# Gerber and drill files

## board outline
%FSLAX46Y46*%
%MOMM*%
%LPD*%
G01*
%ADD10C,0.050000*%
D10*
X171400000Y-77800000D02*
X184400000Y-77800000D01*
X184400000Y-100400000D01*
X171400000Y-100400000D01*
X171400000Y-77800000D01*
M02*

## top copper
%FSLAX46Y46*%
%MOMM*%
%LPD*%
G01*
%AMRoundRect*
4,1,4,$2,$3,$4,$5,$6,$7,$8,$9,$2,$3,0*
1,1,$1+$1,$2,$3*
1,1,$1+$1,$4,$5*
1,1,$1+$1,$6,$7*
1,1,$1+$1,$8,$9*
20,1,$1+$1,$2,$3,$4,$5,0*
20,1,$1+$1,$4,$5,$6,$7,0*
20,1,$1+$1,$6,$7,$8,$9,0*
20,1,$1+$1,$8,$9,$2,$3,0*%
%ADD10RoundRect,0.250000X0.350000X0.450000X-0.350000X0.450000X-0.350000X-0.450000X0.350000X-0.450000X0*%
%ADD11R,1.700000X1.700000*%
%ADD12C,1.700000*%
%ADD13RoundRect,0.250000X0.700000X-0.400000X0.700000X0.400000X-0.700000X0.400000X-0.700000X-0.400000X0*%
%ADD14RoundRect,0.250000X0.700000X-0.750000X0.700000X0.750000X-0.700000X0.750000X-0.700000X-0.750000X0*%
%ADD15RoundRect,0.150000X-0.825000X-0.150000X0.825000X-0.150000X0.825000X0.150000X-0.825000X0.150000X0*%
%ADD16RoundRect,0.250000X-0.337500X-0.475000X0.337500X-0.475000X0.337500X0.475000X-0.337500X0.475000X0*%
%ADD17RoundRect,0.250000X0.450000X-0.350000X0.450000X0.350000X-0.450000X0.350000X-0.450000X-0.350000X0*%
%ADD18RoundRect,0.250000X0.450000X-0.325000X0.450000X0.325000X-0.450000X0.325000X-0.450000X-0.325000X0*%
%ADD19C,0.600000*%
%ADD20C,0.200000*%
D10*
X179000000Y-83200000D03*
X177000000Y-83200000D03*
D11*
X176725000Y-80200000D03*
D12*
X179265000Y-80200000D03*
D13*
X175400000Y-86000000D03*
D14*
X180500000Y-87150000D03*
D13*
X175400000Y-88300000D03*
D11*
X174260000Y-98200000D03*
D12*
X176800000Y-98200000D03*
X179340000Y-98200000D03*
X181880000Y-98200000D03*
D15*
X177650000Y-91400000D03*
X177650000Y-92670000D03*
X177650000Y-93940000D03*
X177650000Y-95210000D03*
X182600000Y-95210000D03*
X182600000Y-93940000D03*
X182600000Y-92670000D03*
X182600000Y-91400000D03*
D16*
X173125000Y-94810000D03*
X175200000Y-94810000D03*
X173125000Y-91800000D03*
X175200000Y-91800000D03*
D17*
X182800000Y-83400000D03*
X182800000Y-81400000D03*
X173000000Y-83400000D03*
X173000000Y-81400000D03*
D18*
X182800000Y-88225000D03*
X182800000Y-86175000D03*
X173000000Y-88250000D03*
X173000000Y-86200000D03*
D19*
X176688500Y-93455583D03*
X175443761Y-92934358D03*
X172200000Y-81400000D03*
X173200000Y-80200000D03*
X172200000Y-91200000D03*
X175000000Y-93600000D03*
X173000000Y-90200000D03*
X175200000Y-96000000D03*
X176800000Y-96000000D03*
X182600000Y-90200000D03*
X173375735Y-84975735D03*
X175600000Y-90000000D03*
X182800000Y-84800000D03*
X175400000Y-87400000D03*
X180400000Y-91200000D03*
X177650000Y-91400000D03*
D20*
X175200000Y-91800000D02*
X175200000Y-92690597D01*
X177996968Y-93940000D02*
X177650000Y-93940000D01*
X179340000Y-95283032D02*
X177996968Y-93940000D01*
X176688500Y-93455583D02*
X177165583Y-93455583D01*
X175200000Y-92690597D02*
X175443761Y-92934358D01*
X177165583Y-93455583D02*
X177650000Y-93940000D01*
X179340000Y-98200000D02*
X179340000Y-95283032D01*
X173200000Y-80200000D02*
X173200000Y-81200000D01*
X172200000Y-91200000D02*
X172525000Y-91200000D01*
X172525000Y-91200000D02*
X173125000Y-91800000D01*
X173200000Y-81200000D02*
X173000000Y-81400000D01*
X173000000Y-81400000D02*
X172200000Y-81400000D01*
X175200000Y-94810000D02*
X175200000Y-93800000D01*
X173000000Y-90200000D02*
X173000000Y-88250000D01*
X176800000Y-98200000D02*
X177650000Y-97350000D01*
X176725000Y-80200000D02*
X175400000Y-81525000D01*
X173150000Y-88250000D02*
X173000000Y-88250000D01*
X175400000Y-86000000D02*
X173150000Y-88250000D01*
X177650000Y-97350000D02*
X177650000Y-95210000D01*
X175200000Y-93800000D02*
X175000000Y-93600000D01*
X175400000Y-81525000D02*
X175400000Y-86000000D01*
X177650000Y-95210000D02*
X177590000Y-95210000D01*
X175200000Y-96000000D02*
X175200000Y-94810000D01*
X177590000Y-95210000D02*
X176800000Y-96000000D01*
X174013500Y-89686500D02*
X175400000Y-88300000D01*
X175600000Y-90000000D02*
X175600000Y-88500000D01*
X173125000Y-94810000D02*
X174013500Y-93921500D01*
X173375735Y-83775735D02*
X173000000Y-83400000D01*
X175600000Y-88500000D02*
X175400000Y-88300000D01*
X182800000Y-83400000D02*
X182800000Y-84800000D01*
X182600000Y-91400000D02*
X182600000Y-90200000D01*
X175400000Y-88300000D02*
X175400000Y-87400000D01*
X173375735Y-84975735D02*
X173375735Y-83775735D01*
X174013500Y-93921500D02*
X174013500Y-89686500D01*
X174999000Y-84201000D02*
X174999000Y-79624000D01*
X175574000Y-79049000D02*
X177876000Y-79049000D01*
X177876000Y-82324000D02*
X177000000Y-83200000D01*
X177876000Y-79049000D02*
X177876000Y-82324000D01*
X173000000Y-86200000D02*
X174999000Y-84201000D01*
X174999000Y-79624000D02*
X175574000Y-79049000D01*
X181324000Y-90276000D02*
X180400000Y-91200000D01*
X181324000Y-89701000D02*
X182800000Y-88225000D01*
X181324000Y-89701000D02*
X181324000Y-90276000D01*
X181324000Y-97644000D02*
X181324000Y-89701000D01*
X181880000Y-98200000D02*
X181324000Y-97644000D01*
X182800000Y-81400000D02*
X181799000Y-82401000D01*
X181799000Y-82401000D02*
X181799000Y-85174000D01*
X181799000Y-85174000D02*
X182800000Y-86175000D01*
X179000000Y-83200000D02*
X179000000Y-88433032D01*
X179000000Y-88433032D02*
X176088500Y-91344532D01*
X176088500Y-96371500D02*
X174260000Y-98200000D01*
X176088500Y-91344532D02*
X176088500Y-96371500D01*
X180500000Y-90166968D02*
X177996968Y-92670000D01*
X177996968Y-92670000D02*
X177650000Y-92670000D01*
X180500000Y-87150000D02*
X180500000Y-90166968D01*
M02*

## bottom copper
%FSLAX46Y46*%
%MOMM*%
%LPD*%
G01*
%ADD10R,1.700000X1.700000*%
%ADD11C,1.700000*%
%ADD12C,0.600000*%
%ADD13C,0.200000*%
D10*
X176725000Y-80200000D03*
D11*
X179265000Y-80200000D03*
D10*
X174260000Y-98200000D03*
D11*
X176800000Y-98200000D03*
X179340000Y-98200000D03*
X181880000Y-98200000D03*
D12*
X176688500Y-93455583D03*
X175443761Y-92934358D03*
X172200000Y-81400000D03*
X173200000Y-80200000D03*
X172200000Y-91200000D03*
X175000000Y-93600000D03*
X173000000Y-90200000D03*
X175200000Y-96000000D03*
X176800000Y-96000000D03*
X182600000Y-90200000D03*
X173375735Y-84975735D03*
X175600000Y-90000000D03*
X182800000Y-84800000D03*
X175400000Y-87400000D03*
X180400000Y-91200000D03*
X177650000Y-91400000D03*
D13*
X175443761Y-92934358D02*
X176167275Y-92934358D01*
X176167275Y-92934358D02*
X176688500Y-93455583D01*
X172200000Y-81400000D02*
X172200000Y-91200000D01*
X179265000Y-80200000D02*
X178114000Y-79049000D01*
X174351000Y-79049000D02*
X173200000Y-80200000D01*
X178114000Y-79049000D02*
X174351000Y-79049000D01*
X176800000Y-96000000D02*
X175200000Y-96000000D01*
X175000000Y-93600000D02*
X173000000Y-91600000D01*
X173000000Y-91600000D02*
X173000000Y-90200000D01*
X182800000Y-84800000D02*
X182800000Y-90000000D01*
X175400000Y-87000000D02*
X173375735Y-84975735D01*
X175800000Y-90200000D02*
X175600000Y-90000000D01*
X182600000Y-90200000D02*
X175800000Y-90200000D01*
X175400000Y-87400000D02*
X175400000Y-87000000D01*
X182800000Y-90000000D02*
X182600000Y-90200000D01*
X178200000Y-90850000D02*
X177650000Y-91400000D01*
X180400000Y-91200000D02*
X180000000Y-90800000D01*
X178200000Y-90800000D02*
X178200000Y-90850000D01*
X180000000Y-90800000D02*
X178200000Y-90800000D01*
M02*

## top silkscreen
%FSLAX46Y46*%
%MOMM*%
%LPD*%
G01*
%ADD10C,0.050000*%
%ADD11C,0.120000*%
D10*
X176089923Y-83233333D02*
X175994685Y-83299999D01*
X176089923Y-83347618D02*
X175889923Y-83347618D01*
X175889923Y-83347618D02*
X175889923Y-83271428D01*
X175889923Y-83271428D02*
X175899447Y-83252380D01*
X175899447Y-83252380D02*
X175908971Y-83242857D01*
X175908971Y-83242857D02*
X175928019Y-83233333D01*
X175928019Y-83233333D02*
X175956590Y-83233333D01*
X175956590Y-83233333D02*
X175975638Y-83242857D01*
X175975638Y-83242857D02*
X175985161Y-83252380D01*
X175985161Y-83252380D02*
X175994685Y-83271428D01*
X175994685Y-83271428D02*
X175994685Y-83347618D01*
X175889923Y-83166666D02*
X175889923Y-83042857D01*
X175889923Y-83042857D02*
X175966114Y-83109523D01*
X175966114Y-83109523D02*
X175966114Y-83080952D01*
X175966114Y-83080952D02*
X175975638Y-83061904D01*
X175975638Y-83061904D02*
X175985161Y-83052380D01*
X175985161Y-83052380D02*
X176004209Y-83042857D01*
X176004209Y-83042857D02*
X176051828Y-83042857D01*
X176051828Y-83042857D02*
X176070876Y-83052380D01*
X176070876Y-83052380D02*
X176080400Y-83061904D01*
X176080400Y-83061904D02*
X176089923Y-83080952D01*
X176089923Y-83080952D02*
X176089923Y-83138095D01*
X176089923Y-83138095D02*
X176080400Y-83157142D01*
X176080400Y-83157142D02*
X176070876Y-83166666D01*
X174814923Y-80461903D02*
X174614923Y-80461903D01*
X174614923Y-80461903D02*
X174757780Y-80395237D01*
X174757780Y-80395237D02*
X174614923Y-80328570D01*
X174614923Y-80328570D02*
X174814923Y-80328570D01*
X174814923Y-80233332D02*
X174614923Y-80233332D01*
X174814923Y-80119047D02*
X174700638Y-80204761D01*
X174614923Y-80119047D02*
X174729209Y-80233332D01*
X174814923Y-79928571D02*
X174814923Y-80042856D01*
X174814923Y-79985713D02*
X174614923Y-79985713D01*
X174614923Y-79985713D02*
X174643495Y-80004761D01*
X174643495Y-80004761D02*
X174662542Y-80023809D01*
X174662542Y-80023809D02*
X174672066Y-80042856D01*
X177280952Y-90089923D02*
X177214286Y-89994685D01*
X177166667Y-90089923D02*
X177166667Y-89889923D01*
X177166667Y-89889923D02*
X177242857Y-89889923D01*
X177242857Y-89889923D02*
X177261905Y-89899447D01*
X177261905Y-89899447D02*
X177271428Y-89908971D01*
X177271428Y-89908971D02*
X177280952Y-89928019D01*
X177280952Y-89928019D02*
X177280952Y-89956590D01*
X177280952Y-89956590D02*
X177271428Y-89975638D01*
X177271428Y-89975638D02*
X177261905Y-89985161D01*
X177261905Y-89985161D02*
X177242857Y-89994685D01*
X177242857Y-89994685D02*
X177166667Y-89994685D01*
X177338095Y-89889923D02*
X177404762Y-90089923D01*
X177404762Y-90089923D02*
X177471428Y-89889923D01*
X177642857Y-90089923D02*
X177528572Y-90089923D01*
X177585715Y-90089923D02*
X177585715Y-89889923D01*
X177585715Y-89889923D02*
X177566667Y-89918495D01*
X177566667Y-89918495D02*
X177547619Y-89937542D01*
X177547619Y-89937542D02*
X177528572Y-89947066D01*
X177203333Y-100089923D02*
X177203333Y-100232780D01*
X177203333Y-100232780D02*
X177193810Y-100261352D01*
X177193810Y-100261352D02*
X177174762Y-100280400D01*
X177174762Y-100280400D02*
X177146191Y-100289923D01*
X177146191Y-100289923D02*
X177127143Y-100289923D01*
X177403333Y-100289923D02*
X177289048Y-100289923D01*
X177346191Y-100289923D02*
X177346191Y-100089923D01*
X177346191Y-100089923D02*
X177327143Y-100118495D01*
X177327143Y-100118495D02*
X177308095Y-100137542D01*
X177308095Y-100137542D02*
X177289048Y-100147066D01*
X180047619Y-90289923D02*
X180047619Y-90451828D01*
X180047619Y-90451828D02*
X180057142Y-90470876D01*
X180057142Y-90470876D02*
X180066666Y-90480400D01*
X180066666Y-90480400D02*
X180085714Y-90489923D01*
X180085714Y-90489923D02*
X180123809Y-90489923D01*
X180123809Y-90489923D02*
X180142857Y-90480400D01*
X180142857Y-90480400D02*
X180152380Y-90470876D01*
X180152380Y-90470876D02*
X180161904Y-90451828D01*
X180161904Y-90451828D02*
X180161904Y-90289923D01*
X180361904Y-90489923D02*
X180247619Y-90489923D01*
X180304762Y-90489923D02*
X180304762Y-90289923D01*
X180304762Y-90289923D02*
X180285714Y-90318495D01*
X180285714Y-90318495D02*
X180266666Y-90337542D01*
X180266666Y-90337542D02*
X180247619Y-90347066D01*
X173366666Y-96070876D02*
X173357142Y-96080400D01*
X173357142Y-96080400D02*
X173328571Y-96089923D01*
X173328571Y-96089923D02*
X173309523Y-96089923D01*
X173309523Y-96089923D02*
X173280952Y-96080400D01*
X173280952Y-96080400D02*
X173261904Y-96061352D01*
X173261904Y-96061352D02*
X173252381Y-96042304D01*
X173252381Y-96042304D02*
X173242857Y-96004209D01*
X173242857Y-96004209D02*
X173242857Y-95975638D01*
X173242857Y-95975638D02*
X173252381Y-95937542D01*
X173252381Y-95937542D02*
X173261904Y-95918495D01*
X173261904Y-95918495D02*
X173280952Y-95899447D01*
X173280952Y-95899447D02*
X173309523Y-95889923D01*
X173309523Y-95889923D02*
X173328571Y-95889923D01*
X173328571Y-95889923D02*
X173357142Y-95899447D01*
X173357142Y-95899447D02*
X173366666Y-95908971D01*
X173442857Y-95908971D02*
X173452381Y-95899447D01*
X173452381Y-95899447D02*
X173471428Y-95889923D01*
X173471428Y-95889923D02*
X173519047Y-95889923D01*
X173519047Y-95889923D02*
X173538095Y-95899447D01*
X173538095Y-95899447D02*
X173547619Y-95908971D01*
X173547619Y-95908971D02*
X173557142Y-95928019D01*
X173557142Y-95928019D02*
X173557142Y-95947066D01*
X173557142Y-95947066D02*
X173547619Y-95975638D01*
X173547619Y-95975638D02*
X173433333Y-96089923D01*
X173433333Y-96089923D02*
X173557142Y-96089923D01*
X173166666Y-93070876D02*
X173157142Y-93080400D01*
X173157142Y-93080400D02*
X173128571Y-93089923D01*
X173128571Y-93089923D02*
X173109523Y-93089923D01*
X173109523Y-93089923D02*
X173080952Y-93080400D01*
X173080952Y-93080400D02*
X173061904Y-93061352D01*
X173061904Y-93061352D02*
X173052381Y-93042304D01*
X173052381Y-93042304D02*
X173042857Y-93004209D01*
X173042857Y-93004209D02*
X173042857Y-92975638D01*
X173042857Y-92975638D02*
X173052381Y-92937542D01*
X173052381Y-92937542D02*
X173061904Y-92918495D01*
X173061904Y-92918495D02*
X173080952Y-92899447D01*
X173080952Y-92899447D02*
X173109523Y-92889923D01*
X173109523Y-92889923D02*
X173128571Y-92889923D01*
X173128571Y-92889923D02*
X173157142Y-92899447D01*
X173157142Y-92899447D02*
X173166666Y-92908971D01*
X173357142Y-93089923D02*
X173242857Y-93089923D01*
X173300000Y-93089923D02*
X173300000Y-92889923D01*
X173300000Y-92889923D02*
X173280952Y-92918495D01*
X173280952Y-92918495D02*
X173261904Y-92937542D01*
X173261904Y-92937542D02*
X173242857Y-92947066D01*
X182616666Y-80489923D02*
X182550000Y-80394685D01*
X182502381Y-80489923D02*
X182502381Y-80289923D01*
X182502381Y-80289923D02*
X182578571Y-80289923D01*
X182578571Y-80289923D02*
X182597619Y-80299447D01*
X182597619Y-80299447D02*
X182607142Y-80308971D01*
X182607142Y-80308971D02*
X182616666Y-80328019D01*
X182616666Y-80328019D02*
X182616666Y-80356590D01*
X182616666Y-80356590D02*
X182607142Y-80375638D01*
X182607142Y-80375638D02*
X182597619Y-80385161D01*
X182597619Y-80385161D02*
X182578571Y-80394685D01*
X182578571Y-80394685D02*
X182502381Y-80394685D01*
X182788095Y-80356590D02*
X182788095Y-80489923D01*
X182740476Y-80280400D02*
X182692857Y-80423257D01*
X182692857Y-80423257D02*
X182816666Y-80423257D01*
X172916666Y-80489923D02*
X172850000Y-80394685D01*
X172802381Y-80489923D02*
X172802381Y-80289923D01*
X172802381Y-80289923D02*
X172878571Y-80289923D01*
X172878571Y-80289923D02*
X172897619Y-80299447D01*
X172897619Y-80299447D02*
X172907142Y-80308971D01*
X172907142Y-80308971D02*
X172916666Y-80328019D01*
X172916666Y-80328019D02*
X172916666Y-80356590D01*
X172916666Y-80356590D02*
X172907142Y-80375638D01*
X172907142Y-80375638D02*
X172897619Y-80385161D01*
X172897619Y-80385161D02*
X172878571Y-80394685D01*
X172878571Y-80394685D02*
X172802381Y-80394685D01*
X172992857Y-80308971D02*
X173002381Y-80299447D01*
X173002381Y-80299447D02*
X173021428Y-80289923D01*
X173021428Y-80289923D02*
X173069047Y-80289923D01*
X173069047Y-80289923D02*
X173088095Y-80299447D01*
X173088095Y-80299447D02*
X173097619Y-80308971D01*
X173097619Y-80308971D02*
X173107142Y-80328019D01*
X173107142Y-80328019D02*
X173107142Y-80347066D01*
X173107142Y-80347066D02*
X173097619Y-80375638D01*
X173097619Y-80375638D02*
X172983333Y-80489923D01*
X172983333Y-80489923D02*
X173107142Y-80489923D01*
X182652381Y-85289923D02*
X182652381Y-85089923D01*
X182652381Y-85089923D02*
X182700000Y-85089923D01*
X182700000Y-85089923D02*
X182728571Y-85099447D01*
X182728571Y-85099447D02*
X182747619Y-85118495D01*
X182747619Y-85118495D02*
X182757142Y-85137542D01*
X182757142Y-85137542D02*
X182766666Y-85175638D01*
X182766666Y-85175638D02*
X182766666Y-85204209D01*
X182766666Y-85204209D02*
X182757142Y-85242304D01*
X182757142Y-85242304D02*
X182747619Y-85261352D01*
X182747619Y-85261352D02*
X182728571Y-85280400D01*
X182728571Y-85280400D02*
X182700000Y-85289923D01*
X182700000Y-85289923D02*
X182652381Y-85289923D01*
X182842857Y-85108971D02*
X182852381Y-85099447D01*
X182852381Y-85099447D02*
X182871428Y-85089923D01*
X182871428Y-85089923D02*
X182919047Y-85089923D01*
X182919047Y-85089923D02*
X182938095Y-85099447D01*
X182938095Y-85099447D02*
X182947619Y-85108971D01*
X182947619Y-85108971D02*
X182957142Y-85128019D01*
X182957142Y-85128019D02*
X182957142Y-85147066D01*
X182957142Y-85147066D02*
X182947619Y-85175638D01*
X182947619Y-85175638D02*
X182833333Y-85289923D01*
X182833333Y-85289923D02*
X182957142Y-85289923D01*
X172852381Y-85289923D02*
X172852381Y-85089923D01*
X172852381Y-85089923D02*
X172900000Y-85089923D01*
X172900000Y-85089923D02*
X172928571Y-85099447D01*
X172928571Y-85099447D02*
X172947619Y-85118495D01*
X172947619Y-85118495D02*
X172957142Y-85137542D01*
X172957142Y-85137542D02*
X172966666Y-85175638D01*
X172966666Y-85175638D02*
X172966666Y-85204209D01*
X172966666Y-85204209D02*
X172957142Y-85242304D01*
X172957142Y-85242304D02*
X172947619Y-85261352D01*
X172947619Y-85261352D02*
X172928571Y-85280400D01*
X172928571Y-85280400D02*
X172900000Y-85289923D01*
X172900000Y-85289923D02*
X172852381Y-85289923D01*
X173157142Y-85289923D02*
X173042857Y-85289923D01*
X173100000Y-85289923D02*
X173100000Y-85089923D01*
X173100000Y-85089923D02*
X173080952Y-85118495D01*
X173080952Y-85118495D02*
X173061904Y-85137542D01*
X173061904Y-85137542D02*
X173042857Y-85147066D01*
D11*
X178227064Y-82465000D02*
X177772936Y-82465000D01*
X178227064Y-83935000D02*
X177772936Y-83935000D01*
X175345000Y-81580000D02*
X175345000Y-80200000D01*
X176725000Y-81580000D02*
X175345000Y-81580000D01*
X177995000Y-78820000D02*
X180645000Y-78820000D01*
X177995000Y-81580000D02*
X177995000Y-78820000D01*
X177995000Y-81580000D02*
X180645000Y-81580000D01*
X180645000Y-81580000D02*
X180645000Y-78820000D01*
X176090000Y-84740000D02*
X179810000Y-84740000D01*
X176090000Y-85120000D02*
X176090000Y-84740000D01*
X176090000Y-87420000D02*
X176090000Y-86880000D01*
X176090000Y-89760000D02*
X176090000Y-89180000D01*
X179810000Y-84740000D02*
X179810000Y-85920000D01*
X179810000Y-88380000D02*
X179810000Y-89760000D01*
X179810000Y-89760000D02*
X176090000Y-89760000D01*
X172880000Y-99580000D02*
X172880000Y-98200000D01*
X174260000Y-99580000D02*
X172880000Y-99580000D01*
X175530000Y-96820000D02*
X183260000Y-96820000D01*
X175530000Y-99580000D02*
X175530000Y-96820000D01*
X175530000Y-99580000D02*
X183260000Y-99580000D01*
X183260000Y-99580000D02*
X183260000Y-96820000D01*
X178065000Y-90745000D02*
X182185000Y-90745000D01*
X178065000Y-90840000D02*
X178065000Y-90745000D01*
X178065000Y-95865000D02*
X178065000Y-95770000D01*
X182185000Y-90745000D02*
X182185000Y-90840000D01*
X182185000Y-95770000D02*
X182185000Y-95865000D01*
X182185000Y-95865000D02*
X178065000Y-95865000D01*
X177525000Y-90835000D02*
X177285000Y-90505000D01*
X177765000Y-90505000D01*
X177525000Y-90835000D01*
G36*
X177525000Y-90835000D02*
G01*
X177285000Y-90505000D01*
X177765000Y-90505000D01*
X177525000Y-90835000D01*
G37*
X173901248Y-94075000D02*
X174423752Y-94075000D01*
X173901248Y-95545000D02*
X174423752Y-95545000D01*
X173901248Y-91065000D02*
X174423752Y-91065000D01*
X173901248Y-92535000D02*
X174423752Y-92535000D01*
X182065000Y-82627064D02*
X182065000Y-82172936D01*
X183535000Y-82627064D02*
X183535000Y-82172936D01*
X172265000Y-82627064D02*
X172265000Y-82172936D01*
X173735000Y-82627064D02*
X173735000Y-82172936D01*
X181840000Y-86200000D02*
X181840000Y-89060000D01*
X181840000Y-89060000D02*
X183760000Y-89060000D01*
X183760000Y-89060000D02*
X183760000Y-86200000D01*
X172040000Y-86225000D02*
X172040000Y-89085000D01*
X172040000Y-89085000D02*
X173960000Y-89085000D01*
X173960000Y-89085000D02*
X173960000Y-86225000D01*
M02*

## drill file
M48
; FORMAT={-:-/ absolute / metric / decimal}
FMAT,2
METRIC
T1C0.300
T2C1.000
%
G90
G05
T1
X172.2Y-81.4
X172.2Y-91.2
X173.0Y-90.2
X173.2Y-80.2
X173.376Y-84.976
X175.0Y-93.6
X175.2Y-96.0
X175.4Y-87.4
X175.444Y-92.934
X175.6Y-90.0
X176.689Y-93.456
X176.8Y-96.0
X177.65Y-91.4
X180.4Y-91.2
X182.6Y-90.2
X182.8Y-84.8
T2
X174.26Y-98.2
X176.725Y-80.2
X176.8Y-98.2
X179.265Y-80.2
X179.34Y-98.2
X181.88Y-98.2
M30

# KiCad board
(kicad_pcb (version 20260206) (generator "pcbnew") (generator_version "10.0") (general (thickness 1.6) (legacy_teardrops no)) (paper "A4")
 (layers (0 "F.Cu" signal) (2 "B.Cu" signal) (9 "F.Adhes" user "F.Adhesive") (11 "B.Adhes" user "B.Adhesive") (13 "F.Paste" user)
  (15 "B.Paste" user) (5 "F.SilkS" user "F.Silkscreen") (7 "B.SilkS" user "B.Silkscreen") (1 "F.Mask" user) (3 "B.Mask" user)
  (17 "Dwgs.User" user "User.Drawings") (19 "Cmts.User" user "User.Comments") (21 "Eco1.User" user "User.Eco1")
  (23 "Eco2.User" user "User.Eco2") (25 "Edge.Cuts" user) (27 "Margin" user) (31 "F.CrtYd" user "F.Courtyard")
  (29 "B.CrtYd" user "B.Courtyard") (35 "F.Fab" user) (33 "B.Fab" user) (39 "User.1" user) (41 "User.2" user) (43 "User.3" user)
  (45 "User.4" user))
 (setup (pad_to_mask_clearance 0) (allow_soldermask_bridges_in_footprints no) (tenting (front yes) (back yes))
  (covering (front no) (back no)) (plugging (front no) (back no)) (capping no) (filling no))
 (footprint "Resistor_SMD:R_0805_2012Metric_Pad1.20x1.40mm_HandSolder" (layer "F.Cu") (at 178 83.2 180)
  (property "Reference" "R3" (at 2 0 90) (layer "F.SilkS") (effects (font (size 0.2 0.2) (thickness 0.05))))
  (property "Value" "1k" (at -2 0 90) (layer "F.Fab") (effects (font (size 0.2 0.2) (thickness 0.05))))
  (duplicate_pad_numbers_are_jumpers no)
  (fp_line (start -0.227064 0.735) (end 0.227064 0.735) (stroke (width 0.12) (type solid)) (layer "F.SilkS"))
  (fp_line (start -0.227064 -0.735) (end 0.227064 -0.735) (stroke (width 0.12) (type solid)) (layer "F.SilkS"))
  (pad "1" smd roundrect (at -1 0 180) (size 1.2 1.4) (layers "F.Cu" "F.Mask" "F.Paste") (roundrect_rratio 0.208333) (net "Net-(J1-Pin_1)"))
  (pad "2" smd roundrect (at 1 0 180) (size 1.2 1.4) (layers "F.Cu" "F.Mask" "F.Paste") (roundrect_rratio 0.208333) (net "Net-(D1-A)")))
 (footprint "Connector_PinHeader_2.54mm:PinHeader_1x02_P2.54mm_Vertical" (layer "F.Cu") (at 176.725 80.2 90)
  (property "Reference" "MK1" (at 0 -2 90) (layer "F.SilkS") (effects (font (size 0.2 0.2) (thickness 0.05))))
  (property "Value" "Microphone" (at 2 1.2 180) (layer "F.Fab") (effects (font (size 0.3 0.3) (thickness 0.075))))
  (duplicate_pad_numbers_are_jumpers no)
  (fp_line (start -1.38 -1.38) (end 0 -1.38) (stroke (width 0.12) (type solid)) (layer "F.SilkS"))
  (fp_line (start -1.38 0) (end -1.38 -1.38) (stroke (width 0.12) (type solid)) (layer "F.SilkS"))
  (fp_line (start 1.38 1.27) (end 1.38 3.92) (stroke (width 0.12) (type solid)) (layer "F.SilkS"))
  (fp_line (start -1.38 1.27) (end 1.38 1.27) (stroke (width 0.12) (type solid)) (layer "F.SilkS"))
  (fp_line (start -1.38 1.27) (end -1.38 3.92) (stroke (width 0.12) (type solid)) (layer "F.SilkS"))
  (fp_line (start -1.38 3.92) (end 1.38 3.92) (stroke (width 0.12) (type solid)) (layer "F.SilkS"))
  (pad "1" thru_hole rect (at 0 0 90) (size 1.7 1.7) (drill 1) (layers "*.Cu" "*.Mask") (remove_unused_layers no) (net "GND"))
  (pad "2" thru_hole circle (at 0 2.54 90) (size 1.7 1.7) (drill 1) (layers "*.Cu" "*.Mask") (remove_unused_layers no) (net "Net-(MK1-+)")))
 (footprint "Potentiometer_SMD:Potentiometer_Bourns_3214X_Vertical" (layer "F.Cu") (at 177.95 87.15 90)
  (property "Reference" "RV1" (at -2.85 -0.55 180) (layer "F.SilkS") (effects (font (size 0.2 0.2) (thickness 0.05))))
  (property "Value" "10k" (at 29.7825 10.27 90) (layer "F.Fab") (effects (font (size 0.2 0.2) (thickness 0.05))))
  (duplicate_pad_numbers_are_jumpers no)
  (fp_line (start 2.41 -1.86) (end 2.41 1.86) (stroke (width 0.12) (type solid)) (layer "F.SilkS"))
  (fp_line (start 2.03 -1.86) (end 2.41 -1.86) (stroke (width 0.12) (type solid)) (layer "F.SilkS"))
  (fp_line (start -0.27 -1.86) (end 0.27 -1.86) (stroke (width 0.12) (type solid)) (layer "F.SilkS"))
  (fp_line (start -2.61 -1.86) (end -2.03 -1.86) (stroke (width 0.12) (type solid)) (layer "F.SilkS"))
  (fp_line (start 2.41 1.86) (end 1.23 1.86) (stroke (width 0.12) (type solid)) (layer "F.SilkS"))
  (fp_line (start -1.23 1.86) (end -2.61 1.86) (stroke (width 0.12) (type solid)) (layer "F.SilkS"))
  (fp_line (start -2.61 1.86) (end -2.61 -1.86) (stroke (width 0.12) (type solid)) (layer "F.SilkS"))
  (pad "1" smd roundrect (at 1.15 -2.55 90) (size 1.3 1.9) (layers "F.Cu" "F.Mask" "F.Paste") (roundrect_rratio 0.192308) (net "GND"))
  (pad "2" smd roundrect (at 0 2.55 90) (size 2 1.9) (layers "F.Cu" "F.Mask" "F.Paste") (roundrect_rratio 0.131579) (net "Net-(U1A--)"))
  (pad "3" smd roundrect (at -1.15 -2.55 90) (size 1.3 1.9) (layers "F.Cu" "F.Mask" "F.Paste") (roundrect_rratio 0.192308) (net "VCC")))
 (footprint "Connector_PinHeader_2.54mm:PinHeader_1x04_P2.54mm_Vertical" (layer "F.Cu") (at 174.26 98.2 90)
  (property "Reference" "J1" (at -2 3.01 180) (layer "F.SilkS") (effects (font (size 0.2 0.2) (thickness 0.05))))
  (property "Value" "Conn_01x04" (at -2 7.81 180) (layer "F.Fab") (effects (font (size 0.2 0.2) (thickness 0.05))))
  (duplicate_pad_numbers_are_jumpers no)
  (fp_line (start -1.38 -1.38) (end 0 -1.38) (stroke (width 0.12) (type solid)) (layer "F.SilkS"))
  (fp_line (start -1.38 0) (end -1.38 -1.38) (stroke (width 0.12) (type solid)) (layer "F.SilkS"))
  (fp_line (start 1.38 1.27) (end 1.38 9) (stroke (width 0.12) (type solid)) (layer "F.SilkS"))
  (fp_line (start -1.38 1.27) (end 1.38 1.27) (stroke (width 0.12) (type solid)) (layer "F.SilkS"))
  (fp_line (start -1.38 1.27) (end -1.38 9) (stroke (width 0.12) (type solid)) (layer "F.SilkS"))
  (fp_line (start -1.38 9) (end 1.38 9) (stroke (width 0.12) (type solid)) (layer "F.SilkS"))
  (pad "1" thru_hole rect (at 0 0 90) (size 1.7 1.7) (drill 1) (layers "*.Cu" "*.Mask") (remove_unused_layers no) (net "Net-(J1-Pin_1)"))
  (pad "2" thru_hole circle (at 0 2.54 90) (size 1.7 1.7) (drill 1) (layers "*.Cu" "*.Mask") (remove_unused_layers no) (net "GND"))
  (pad "3" thru_hole circle (at 0 5.08 90) (size 1.7 1.7) (drill 1) (layers "*.Cu" "*.Mask") (remove_unused_layers no)
   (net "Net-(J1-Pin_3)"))
  (pad "4" thru_hole circle (at 0 7.62 90) (size 1.7 1.7) (drill 1) (layers "*.Cu" "*.Mask") (remove_unused_layers no) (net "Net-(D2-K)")))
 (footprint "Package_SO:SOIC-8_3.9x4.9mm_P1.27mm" (layer "F.Cu") (at 180.125 93.305)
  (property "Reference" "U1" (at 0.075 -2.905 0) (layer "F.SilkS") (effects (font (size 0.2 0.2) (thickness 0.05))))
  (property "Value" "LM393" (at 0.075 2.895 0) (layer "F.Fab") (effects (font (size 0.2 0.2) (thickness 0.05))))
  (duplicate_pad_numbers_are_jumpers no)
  (fp_line (start -2.06 -2.56) (end 2.06 -2.56) (stroke (width 0.12) (type solid)) (layer "F.SilkS"))
  (fp_line (start -2.06 -2.465) (end -2.06 -2.56) (stroke (width 0.12) (type solid)) (layer "F.SilkS"))
  (fp_line (start -2.06 2.56) (end -2.06 2.465) (stroke (width 0.12) (type solid)) (layer "F.SilkS"))
  (fp_line (start 2.06 -2.56) (end 2.06 -2.465) (stroke (width 0.12) (type solid)) (layer "F.SilkS"))
  (fp_line (start 2.06 2.465) (end 2.06 2.56) (stroke (width 0.12) (type solid)) (layer "F.SilkS"))
  (fp_line (start 2.06 2.56) (end -2.06 2.56) (stroke (width 0.12) (type solid)) (layer "F.SilkS"))
  (fp_poly (pts (xy -2.6 -2.47) (xy -2.84 -2.8) (xy -2.36 -2.8)) (stroke (width 0.12) (type solid)) (fill yes) (layer "F.SilkS"))
  (pad "1" smd roundrect (at -2.475 -1.905) (size 1.95 0.6) (layers "F.Cu" "F.Mask" "F.Paste") (roundrect_rratio 0.25) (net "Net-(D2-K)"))
  (pad "2" smd roundrect (at -2.475 -0.635) (size 1.95 0.6) (layers "F.Cu" "F.Mask" "F.Paste") (roundrect_rratio 0.25) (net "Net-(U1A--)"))
  (pad "3" smd roundrect (at -2.475 0.635) (size 1.95 0.6) (layers "F.Cu" "F.Mask" "F.Paste") (roundrect_rratio 0.25) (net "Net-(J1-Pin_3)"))
  (pad "4" smd roundrect (at -2.475 1.905) (size 1.95 0.6) (layers "F.Cu" "F.Mask" "F.Paste") (roundrect_rratio 0.25) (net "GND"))
  (pad "5" smd roundrect (at 2.475 1.905) (size 1.95 0.6) (layers "F.Cu" "F.Mask" "F.Paste") (roundrect_rratio 0.25))
  (pad "6" smd roundrect (at 2.475 0.635) (size 1.95 0.6) (layers "F.Cu" "F.Mask" "F.Paste") (roundrect_rratio 0.25))
  (pad "7" smd roundrect (at 2.475 -0.635) (size 1.95 0.6) (layers "F.Cu" "F.Mask" "F.Paste") (roundrect_rratio 0.25))
  (pad "8" smd roundrect (at 2.475 -1.905) (size 1.95 0.6) (layers "F.Cu" "F.Mask" "F.Paste") (roundrect_rratio 0.25) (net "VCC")))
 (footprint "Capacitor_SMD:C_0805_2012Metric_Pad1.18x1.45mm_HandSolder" (layer "F.Cu") (at 174.1625 94.81)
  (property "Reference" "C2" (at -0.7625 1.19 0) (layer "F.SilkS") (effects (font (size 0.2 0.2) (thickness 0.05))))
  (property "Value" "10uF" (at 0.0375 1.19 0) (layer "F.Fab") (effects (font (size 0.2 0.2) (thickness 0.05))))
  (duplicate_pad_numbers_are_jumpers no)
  (fp_line (start -0.261252 -0.735) (end 0.261252 -0.735) (stroke (width 0.12) (type solid)) (layer "F.SilkS"))
  (fp_line (start -0.261252 0.735) (end 0.261252 0.735) (stroke (width 0.12) (type solid)) (layer "F.SilkS"))
  (pad "1" smd roundrect (at -1.0375 0) (size 1.175 1.45) (layers "F.Cu" "F.Mask" "F.Paste") (roundrect_rratio 0.212766) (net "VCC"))
  (pad "2" smd roundrect (at 1.0375 0) (size 1.175 1.45) (layers "F.Cu" "F.Mask" "F.Paste") (roundrect_rratio 0.212766) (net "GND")))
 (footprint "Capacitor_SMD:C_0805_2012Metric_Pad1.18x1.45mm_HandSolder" (layer "F.Cu") (at 174.1625 91.8)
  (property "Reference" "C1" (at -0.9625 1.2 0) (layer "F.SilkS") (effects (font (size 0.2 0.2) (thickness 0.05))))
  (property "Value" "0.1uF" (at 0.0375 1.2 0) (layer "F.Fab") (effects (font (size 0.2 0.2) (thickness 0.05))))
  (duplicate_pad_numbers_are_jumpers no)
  (fp_line (start -0.261252 -0.735) (end 0.261252 -0.735) (stroke (width 0.12) (type solid)) (layer "F.SilkS"))
  (fp_line (start -0.261252 0.735) (end 0.261252 0.735) (stroke (width 0.12) (type solid)) (layer "F.SilkS"))
  (pad "1" smd roundrect (at -1.0375 0) (size 1.175 1.45) (layers "F.Cu" "F.Mask" "F.Paste") (roundrect_rratio 0.212766) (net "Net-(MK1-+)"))
  (pad "2" smd roundrect (at 1.0375 0) (size 1.175 1.45) (layers "F.Cu" "F.Mask" "F.Paste") (roundrect_rratio 0.212766)
   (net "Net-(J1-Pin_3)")))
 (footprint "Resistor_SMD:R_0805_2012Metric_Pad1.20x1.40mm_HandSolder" (layer "F.Cu") (at 182.8 82.4 90)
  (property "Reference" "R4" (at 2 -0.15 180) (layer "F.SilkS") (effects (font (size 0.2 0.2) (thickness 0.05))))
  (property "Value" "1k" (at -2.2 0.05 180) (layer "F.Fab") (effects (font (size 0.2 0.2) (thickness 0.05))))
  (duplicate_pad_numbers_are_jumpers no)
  (fp_line (start -0.227064 -0.735) (end 0.227064 -0.735) (stroke (width 0.12) (type solid)) (layer "F.SilkS"))
  (fp_line (start -0.227064 0.735) (end 0.227064 0.735) (stroke (width 0.12) (type solid)) (layer "F.SilkS"))
  (pad "1" smd roundrect (at -1 0 90) (size 1.2 1.4) (layers "F.Cu" "F.Mask" "F.Paste") (roundrect_rratio 0.208333) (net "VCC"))
  (pad "2" smd roundrect (at 1 0 90) (size 1.2 1.4) (layers "F.Cu" "F.Mask" "F.Paste") (roundrect_rratio 0.208333) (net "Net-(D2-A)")))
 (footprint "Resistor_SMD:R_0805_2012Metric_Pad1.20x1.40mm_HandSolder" (layer "F.Cu") (at 173 82.4 90)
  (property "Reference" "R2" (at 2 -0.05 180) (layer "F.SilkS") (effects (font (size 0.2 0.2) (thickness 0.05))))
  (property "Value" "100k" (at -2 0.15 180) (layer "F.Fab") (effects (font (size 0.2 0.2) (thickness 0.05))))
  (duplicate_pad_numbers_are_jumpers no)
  (fp_line (start -0.227064 -0.735) (end 0.227064 -0.735) (stroke (width 0.12) (type solid)) (layer "F.SilkS"))
  (fp_line (start -0.227064 0.735) (end 0.227064 0.735) (stroke (width 0.12) (type solid)) (layer "F.SilkS"))
  (pad "1" smd roundrect (at -1 0 90) (size 1.2 1.4) (layers "F.Cu" "F.Mask" "F.Paste") (roundrect_rratio 0.208333) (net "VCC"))
  (pad "2" smd roundrect (at 1 0 90) (size 1.2 1.4) (layers "F.Cu" "F.Mask" "F.Paste") (roundrect_rratio 0.208333) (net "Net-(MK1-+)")))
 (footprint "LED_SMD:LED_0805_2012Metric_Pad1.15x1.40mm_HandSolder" (layer "F.Cu") (at 182.8 87.2 90)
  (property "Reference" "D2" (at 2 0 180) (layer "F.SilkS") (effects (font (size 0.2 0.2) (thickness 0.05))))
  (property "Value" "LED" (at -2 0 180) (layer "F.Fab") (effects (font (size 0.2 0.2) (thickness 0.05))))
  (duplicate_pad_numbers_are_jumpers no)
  (fp_line (start 1 -0.96) (end -1.86 -0.96) (stroke (width 0.12) (type solid)) (layer "F.SilkS"))
  (fp_line (start -1.86 -0.96) (end -1.86 0.96) (stroke (width 0.12) (type solid)) (layer "F.SilkS"))
  (fp_line (start -1.86 0.96) (end 1 0.96) (stroke (width 0.12) (type solid)) (layer "F.SilkS"))
  (pad "1" smd roundrect (at -1.025 0 90) (size 1.15 1.4) (layers "F.Cu" "F.Mask" "F.Paste") (roundrect_rratio 0.217391) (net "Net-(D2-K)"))
  (pad "2" smd roundrect (at 1.025 0 90) (size 1.15 1.4) (layers "F.Cu" "F.Mask" "F.Paste") (roundrect_rratio 0.217391) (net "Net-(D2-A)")))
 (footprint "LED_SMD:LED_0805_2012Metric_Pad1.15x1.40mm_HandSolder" (layer "F.Cu") (at 173 87.225 90)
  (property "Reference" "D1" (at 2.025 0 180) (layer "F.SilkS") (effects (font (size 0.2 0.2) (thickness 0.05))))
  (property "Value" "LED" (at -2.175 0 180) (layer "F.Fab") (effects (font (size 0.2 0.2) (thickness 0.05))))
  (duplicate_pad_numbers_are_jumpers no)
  (fp_line (start 1 -0.96) (end -1.86 -0.96) (stroke (width 0.12) (type solid)) (layer "F.SilkS"))
  (fp_line (start -1.86 -0.96) (end -1.86 0.96) (stroke (width 0.12) (type solid)) (layer "F.SilkS"))
  (fp_line (start -1.86 0.96) (end 1 0.96) (stroke (width 0.12) (type solid)) (layer "F.SilkS"))
  (pad "1" smd roundrect (at -1.025 0 90) (size 1.15 1.4) (layers "F.Cu" "F.Mask" "F.Paste") (roundrect_rratio 0.217391) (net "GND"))
  (pad "2" smd roundrect (at 1.025 0 90) (size 1.15 1.4) (layers "F.Cu" "F.Mask" "F.Paste") (roundrect_rratio 0.217391) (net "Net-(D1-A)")))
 (gr_rect (start 171.4 77.8) (end 184.4 100.4) (stroke (width 0.05) (type default)) (fill no) (layer "Edge.Cuts"))
 (segment (start 175.2 91.8) (end 175.2 92.690597) (width 0.2) (layer "F.Cu") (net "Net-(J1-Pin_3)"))
 (segment (start 177.996968 93.94) (end 177.65 93.94) (width 0.2) (layer "F.Cu") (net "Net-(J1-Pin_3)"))
 (segment (start 179.34 95.283032) (end 177.996968 93.94) (width 0.2) (layer "F.Cu") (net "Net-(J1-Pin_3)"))
 (segment (start 176.6885 93.455583) (end 177.165583 93.455583) (width 0.2) (layer "F.Cu") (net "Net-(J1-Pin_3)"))
 (segment (start 175.2 92.690597) (end 175.443761 92.934358) (width 0.2) (layer "F.Cu") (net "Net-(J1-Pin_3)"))
 (segment (start 177.165583 93.455583) (end 177.65 93.94) (width 0.2) (layer "F.Cu") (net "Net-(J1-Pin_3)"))
 (segment (start 179.34 98.2) (end 179.34 95.283032) (width 0.2) (layer "F.Cu") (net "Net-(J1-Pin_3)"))
 (via (at 176.6885 93.455583) (size 0.6) (drill 0.3) (layers "F.Cu" "B.Cu") (capping no) (covering (front no) (back no))
  (plugging (front no) (back no)) (filling no) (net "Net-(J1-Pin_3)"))
 (via (at 175.443761 92.934358) (size 0.6) (drill 0.3) (layers "F.Cu" "B.Cu") (capping no) (covering (front no) (back no))
  (plugging (front no) (back no)) (filling no) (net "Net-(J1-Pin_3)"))
 (segment (start 175.443761 92.934358) (end 176.167275 92.934358) (width 0.2) (layer "B.Cu") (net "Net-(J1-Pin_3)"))
 (segment (start 176.167275 92.934358) (end 176.6885 93.455583) (width 0.2) (layer "B.Cu") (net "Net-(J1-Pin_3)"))
 (segment (start 173.2 80.2) (end 173.2 81.2) (width 0.2) (layer "F.Cu") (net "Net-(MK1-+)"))
 (segment (start 172.2 91.2) (end 172.525 91.2) (width 0.2) (layer "F.Cu") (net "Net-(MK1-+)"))
 (segment (start 172.525 91.2) (end 173.125 91.8) (width 0.2) (layer "F.Cu") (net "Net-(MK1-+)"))
 (segment (start 173.2 81.2) (end 173 81.4) (width 0.2) (layer "F.Cu") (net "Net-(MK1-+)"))
 (segment (start 173 81.4) (end 172.2 81.4) (width 0.2) (layer "F.Cu") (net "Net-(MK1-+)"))
 (via (at 172.2 81.4) (size 0.6) (drill 0.3) (layers "F.Cu" "B.Cu") (capping no) (covering (front no) (back no))
  (plugging (front no) (back no)) (filling no) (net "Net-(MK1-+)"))
 (via (at 173.2 80.2) (size 0.6) (drill 0.3) (layers "F.Cu" "B.Cu") (capping no) (covering (front no) (back no))
  (plugging (front no) (back no)) (filling no) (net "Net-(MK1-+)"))
 (via (at 172.2 91.2) (size 0.6) (drill 0.3) (layers "F.Cu" "B.Cu") (capping no) (covering (front no) (back no))
  (plugging (front no) (back no)) (filling no) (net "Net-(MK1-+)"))
 (segment (start 172.2 81.4) (end 172.2 91.2) (width 0.2) (layer "B.Cu") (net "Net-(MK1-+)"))
 (segment (start 179.265 80.2) (end 178.114 79.049) (width 0.2) (layer "B.Cu") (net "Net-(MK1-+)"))
 (segment (start 174.351 79.049) (end 173.2 80.2) (width 0.2) (layer "B.Cu") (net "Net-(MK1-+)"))
 (segment (start 178.114 79.049) (end 174.351 79.049) (width 0.2) (layer "B.Cu") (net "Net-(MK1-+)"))
 (segment (start 175.2 94.81) (end 175.2 93.8) (width 0.2) (layer "F.Cu") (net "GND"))
 (segment (start 173 90.2) (end 173 88.25) (width 0.2) (layer "F.Cu") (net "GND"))
 (segment (start 176.8 98.2) (end 177.65 97.35) (width 0.2) (layer "F.Cu") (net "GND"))
 (segment (start 176.725 80.2) (end 175.4 81.525) (width 0.2) (layer "F.Cu") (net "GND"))
 (segment (start 173.15 88.25) (end 173 88.25) (width 0.2) (layer "F.Cu") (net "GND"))
 (segment (start 175.4 86) (end 173.15 88.25) (width 0.2) (layer "F.Cu") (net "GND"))
 (segment (start 177.65 97.35) (end 177.65 95.21) (width 0.2) (layer "F.Cu") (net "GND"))
 (segment (start 175.2 93.8) (end 175 93.6) (width 0.2) (layer "F.Cu") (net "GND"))
 (segment (start 175.4 81.525) (end 175.4 86) (width 0.2) (layer "F.Cu") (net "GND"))
 (segment (start 177.65 95.21) (end 177.59 95.21) (width 0.2) (layer "F.Cu") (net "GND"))
 (segment (start 175.2 96) (end 175.2 94.81) (width 0.2) (layer "F.Cu") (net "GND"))
 (segment (start 177.59 95.21) (end 176.8 96) (width 0.2) (layer "F.Cu") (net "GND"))
 (via (at 175 93.6) (size 0.6) (drill 0.3) (layers "F.Cu" "B.Cu") (capping no) (covering (front no) (back no))
  (plugging (front no) (back no)) (filling no) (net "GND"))
 (via (at 173 90.2) (size 0.6) (drill 0.3) (layers "F.Cu" "B.Cu") (capping no) (covering (front no) (back no))
  (plugging (front no) (back no)) (filling no) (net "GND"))
 (via (at 175.2 96) (size 0.6) (drill 0.3) (layers "F.Cu" "B.Cu") (capping no) (covering (front no) (back no))
  (plugging (front no) (back no)) (filling no) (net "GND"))
 (via (at 176.8 96) (size 0.6) (drill 0.3) (layers "F.Cu" "B.Cu") (capping no) (covering (front no) (back no))
  (plugging (front no) (back no)) (filling no) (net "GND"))
 (segment (start 176.8 96) (end 175.2 96) (width 0.2) (layer "B.Cu") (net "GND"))
 (segment (start 175 93.6) (end 173 91.6) (width 0.2) (layer "B.Cu") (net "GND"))
 (segment (start 173 91.6) (end 173 90.2) (width 0.2) (layer "B.Cu") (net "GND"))
 (segment (start 174.0135 89.6865) (end 175.4 88.3) (width 0.2) (layer "F.Cu") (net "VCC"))
 (segment (start 175.6 90) (end 175.6 88.5) (width 0.2) (layer "F.Cu") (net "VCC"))
 (segment (start 173.125 94.81) (end 174.0135 93.9215) (width 0.2) (layer "F.Cu") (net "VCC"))
 (segment (start 173.375735 83.775735) (end 173 83.4) (width 0.2) (layer "F.Cu") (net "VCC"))
 (segment (start 175.6 88.5) (end 175.4 88.3) (width 0.2) (layer "F.Cu") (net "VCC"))
 (segment (start 182.8 83.4) (end 182.8 84.8) (width 0.2) (layer "F.Cu") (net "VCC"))
 (segment (start 182.6 91.4) (end 182.6 90.2) (width 0.2) (layer "F.Cu") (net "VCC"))
 (segment (start 175.4 88.3) (end 175.4 87.4) (width 0.2) (layer "F.Cu") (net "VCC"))
 (segment (start 173.375735 84.975735) (end 173.375735 83.775735) (width 0.2) (layer "F.Cu") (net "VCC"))
 (segment (start 174.0135 93.9215) (end 174.0135 89.6865) (width 0.2) (layer "F.Cu") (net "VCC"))
 (via (at 182.6 90.2) (size 0.6) (drill 0.3) (layers "F.Cu" "B.Cu") (capping no) (covering (front no) (back no))
  (plugging (front no) (back no)) (filling no) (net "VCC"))
 (via (at 173.375735 84.975735) (size 0.6) (drill 0.3) (layers "F.Cu" "B.Cu") (capping no) (covering (front no) (back no))
  (plugging (front no) (back no)) (filling no) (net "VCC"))
 (via (at 175.6 90) (size 0.6) (drill 0.3) (layers "F.Cu" "B.Cu") (capping no) (covering (front no) (back no))
  (plugging (front no) (back no)) (filling no) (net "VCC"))
 (via (at 182.8 84.8) (size 0.6) (drill 0.3) (layers "F.Cu" "B.Cu") (capping no) (covering (front no) (back no))
  (plugging (front no) (back no)) (filling no) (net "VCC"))
 (via (at 175.4 87.4) (size 0.6) (drill 0.3) (layers "F.Cu" "B.Cu") (capping no) (covering (front no) (back no))
  (plugging (front no) (back no)) (filling no) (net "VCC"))
 (segment (start 182.8 84.8) (end 182.8 90) (width 0.2) (layer "B.Cu") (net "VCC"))
 (segment (start 175.4 87) (end 173.375735 84.975735) (width 0.2) (layer "B.Cu") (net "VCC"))
 (segment (start 175.8 90.2) (end 175.6 90) (width 0.2) (layer "B.Cu") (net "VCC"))
 (segment (start 182.6 90.2) (end 175.8 90.2) (width 0.2) (layer "B.Cu") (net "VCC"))
 (segment (start 175.4 87.4) (end 175.4 87) (width 0.2) (layer "B.Cu") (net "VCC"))
 (segment (start 182.8 90) (end 182.6 90.2) (width 0.2) (layer "B.Cu") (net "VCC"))
 (segment (start 174.999 84.201) (end 174.999 79.624) (width 0.2) (layer "F.Cu") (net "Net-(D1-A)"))
 (segment (start 175.574 79.049) (end 177.876 79.049) (width 0.2) (layer "F.Cu") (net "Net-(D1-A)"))
 (segment (start 177.876 82.324) (end 177 83.2) (width 0.2) (layer "F.Cu") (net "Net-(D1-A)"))
 (segment (start 177.876 79.049) (end 177.876 82.324) (width 0.2) (layer "F.Cu") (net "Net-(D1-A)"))
 (segment (start 173 86.2) (end 174.999 84.201) (width 0.2) (layer "F.Cu") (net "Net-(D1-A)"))
 (segment (start 174.999 79.624) (end 175.574 79.049) (width 0.2) (layer "F.Cu") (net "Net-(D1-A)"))
 (segment (start 181.324 90.276) (end 180.4 91.2) (width 0.2) (layer "F.Cu") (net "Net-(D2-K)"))
 (segment (start 181.324 89.701) (end 182.8 88.225) (width 0.2) (layer "F.Cu") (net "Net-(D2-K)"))
 (segment (start 181.324 89.701) (end 181.324 90.276) (width 0.2) (layer "F.Cu") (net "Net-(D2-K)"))
 (segment (start 181.324 97.644) (end 181.324 89.701) (width 0.2) (layer "F.Cu") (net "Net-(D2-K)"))
 (segment (start 181.88 98.2) (end 181.324 97.644) (width 0.2) (layer "F.Cu") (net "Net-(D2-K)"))
 (via (at 180.4 91.2) (size 0.6) (drill 0.3) (layers "F.Cu" "B.Cu") (capping no) (covering (front no) (back no))
  (plugging (front no) (back no)) (filling no) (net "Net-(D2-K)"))
 (via (at 177.65 91.4) (size 0.6) (drill 0.3) (layers "F.Cu" "B.Cu") (capping no) (covering (front no) (back no))
  (plugging (front no) (back no)) (filling no) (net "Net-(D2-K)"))
 (segment (start 178.2 90.85) (end 177.65 91.4) (width 0.2) (layer "B.Cu") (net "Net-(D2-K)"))
 (segment (start 180.4 91.2) (end 180 90.8) (width 0.2) (layer "B.Cu") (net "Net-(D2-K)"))
 (segment (start 178.2 90.8) (end 178.2 90.85) (width 0.2) (layer "B.Cu") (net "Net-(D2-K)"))
 (segment (start 180 90.8) (end 178.2 90.8) (width 0.2) (layer "B.Cu") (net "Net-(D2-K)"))
 (segment (start 182.8 81.4) (end 181.799 82.401) (width 0.2) (layer "F.Cu") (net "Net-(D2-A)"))
 (segment (start 181.799 82.401) (end 181.799 85.174) (width 0.2) (layer "F.Cu") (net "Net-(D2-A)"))
 (segment (start 181.799 85.174) (end 182.8 86.175) (width 0.2) (layer "F.Cu") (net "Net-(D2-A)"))
 (segment (start 179 83.2) (end 179 88.433032) (width 0.2) (layer "F.Cu") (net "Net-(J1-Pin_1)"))
 (segment (start 179 88.433032) (end 176.0885 91.344532) (width 0.2) (layer "F.Cu") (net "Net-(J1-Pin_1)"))
 (segment (start 176.0885 96.3715) (end 174.26 98.2) (width 0.2) (layer "F.Cu") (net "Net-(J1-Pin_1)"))
 (segment (start 176.0885 91.344532) (end 176.0885 96.3715) (width 0.2) (layer "F.Cu") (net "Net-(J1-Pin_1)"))
 (segment (start 180.5 90.166968) (end 177.996968 92.67) (width 0.2) (layer "F.Cu") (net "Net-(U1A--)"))
 (segment (start 177.996968 92.67) (end 177.65 92.67) (width 0.2) (layer "F.Cu") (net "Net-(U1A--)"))
 (segment (start 180.5 87.15) (end 180.5 90.166968) (width 0.2) (layer "F.Cu") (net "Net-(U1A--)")))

